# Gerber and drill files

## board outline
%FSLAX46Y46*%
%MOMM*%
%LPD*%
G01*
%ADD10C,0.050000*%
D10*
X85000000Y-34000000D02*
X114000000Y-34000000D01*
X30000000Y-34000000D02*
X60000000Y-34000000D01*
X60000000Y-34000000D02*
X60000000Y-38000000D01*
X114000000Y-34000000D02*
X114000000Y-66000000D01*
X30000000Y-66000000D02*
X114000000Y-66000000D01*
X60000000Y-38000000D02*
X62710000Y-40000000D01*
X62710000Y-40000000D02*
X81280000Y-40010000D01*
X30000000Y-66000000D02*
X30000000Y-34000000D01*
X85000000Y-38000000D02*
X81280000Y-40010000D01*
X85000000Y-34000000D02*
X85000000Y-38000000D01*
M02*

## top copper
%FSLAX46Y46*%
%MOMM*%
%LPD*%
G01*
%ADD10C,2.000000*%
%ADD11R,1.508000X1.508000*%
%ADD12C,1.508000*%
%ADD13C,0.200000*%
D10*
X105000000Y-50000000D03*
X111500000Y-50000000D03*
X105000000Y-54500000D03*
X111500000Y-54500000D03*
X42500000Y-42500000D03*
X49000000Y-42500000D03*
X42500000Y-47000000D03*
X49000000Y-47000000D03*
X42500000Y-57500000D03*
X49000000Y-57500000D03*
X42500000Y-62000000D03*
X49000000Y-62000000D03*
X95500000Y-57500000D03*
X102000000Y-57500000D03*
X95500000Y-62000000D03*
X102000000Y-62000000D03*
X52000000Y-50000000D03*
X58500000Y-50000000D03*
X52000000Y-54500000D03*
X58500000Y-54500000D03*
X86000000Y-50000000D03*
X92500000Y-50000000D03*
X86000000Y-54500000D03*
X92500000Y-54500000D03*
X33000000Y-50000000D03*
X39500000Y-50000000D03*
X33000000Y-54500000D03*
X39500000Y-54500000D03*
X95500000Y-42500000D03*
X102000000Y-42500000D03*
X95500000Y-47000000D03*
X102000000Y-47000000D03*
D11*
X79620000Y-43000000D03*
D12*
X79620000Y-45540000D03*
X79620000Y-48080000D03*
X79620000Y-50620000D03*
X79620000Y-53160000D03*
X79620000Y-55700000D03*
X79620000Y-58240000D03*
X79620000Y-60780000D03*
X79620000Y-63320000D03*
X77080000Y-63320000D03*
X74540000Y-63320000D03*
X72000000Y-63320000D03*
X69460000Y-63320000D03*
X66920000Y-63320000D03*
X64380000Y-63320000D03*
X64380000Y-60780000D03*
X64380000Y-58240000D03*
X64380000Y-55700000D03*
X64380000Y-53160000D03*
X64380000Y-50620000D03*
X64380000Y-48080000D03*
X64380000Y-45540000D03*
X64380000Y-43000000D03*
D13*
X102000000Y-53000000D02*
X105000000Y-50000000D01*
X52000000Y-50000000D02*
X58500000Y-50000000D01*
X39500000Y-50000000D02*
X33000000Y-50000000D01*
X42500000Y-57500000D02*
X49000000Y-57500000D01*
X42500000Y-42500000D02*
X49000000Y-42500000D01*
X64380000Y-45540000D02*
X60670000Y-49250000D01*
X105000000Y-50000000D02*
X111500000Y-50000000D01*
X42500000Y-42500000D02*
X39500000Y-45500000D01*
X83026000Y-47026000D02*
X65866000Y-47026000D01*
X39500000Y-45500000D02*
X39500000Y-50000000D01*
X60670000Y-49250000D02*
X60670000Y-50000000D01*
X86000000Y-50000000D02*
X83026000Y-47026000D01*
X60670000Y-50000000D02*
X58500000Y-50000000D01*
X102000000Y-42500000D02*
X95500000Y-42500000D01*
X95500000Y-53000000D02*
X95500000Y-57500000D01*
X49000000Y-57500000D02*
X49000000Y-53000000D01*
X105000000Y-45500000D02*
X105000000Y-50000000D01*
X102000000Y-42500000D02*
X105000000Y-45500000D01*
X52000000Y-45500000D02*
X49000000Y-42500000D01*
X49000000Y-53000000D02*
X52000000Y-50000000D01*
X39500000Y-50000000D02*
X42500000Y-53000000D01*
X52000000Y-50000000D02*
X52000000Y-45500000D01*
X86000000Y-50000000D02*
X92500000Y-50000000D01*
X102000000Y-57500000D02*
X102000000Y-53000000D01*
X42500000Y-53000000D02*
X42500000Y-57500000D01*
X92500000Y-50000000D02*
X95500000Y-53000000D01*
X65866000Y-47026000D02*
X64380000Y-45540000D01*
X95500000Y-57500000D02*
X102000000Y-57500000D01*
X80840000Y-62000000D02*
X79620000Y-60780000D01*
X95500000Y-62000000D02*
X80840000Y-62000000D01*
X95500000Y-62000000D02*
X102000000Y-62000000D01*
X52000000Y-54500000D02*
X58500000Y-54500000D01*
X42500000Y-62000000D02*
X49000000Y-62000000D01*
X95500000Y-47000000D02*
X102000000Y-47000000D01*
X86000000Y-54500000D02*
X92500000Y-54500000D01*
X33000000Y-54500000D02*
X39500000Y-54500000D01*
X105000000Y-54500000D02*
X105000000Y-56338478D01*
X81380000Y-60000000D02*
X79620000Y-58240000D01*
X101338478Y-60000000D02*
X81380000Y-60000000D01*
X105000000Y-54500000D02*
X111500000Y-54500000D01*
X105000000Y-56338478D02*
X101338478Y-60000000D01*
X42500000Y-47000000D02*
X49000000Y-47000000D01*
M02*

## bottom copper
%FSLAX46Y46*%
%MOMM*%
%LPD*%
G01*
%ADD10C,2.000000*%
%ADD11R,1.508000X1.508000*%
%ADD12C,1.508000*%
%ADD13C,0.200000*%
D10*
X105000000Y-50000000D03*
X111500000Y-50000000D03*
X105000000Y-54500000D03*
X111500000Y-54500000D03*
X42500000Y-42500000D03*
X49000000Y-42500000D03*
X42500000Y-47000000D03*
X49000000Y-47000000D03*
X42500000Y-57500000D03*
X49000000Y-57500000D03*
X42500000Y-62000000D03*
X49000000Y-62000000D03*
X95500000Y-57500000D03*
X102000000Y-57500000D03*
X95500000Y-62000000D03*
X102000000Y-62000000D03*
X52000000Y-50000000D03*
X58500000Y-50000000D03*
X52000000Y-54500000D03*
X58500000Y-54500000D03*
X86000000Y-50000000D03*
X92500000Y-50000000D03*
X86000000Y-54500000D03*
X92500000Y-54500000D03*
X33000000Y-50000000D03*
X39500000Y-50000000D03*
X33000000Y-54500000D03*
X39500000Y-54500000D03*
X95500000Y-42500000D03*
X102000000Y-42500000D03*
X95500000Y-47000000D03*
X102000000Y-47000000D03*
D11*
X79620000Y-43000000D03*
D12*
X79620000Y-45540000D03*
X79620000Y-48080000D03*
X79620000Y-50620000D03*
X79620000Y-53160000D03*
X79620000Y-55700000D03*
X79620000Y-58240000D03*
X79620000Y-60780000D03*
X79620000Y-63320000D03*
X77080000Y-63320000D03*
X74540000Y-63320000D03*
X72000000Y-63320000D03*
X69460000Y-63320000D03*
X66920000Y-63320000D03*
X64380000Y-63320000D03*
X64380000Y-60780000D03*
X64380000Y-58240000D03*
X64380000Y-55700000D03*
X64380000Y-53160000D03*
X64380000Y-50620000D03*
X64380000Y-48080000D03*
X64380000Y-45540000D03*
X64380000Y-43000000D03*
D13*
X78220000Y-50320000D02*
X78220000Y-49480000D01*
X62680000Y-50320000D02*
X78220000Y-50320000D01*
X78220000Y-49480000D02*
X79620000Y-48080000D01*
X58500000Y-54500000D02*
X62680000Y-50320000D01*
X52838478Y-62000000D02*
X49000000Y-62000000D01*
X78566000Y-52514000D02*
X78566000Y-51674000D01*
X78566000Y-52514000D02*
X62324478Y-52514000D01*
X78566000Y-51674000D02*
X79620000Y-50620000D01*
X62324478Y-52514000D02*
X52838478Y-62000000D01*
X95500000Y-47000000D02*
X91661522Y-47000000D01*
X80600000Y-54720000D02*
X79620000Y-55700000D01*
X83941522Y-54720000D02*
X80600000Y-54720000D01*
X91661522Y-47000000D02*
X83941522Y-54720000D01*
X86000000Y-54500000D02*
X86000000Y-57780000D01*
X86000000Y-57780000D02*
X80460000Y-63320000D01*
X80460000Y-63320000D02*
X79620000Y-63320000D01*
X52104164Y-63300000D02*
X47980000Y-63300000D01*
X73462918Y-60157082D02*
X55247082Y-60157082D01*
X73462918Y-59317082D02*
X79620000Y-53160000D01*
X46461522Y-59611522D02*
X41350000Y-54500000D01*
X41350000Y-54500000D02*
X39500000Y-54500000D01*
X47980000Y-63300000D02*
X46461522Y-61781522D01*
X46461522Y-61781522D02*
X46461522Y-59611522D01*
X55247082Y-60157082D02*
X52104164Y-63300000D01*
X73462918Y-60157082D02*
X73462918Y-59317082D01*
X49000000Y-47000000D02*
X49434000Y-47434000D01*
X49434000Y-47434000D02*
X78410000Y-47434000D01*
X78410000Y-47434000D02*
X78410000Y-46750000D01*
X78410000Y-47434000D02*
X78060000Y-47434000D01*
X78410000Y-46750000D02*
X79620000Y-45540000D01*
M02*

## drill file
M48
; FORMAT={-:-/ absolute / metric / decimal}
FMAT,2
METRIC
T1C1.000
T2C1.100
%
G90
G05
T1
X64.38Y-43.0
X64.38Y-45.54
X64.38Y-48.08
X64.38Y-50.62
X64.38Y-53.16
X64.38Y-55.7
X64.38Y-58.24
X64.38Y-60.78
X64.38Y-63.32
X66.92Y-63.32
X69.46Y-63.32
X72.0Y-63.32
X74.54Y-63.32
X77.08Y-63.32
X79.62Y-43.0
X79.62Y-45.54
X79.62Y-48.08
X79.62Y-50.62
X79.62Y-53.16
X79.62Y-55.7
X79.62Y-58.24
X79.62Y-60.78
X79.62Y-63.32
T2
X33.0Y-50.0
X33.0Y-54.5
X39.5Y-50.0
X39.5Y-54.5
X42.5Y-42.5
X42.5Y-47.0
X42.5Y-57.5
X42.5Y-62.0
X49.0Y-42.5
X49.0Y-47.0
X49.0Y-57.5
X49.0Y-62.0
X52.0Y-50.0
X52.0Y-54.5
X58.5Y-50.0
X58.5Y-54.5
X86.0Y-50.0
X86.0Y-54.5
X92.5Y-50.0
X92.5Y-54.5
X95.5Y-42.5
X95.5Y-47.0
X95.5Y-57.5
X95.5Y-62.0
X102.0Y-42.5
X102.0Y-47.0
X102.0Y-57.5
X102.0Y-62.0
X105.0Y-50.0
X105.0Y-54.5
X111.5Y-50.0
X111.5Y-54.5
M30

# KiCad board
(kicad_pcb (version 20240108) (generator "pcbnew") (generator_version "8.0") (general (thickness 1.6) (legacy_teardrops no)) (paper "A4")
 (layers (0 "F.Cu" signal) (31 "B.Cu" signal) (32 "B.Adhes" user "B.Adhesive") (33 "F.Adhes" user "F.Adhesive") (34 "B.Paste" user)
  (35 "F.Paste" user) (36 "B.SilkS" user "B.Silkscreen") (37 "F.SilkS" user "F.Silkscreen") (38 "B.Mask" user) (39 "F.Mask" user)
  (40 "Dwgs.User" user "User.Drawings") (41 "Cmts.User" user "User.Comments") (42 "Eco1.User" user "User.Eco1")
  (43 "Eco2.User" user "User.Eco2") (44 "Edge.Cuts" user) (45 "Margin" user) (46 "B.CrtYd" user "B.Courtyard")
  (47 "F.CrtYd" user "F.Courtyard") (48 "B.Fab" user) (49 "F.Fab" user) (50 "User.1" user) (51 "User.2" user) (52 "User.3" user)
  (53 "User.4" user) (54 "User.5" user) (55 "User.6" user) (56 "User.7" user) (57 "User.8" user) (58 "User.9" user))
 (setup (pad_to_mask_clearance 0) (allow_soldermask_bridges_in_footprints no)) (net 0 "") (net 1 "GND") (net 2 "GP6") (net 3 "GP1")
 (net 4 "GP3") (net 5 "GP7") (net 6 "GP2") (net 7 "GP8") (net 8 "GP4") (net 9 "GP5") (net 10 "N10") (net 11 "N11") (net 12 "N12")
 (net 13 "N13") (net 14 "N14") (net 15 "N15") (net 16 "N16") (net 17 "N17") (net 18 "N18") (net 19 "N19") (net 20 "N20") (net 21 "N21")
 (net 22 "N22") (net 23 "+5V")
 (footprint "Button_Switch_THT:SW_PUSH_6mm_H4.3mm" (layer "F.Cu") (at 105 50)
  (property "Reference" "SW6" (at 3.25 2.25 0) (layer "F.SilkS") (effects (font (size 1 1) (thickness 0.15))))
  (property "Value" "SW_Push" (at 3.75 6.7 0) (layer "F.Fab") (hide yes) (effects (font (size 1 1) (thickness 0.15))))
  (pad "1" thru_hole circle (at 0 0 90) (size 2 2) (drill 1.1) (layers "*.Cu" "*.Mask") (remove_unused_layers no) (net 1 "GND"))
  (pad "1" thru_hole circle (at 6.5 0 90) (size 2 2) (drill 1.1) (layers "*.Cu" "*.Mask") (remove_unused_layers no) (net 1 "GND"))
  (pad "2" thru_hole circle (at 0 4.5 90) (size 2 2) (drill 1.1) (layers "*.Cu" "*.Mask") (remove_unused_layers no) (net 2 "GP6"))
  (pad "2" thru_hole circle (at 6.5 4.5 90) (size 2 2) (drill 1.1) (layers "*.Cu" "*.Mask") (remove_unused_layers no) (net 2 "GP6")))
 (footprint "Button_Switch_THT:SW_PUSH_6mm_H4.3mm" (layer "F.Cu") (at 42.5 42.5)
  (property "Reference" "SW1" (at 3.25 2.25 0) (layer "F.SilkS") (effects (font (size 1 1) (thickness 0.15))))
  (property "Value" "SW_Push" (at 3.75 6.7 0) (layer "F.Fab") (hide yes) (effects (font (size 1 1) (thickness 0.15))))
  (pad "1" thru_hole circle (at 0 0 90) (size 2 2) (drill 1.1) (layers "*.Cu" "*.Mask") (remove_unused_layers no) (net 1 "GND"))
  (pad "1" thru_hole circle (at 6.5 0 90) (size 2 2) (drill 1.1) (layers "*.Cu" "*.Mask") (remove_unused_layers no) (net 1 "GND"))
  (pad "2" thru_hole circle (at 0 4.5 90) (size 2 2) (drill 1.1) (layers "*.Cu" "*.Mask") (remove_unused_layers no) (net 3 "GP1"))
  (pad "2" thru_hole circle (at 6.5 4.5 90) (size 2 2) (drill 1.1) (layers "*.Cu" "*.Mask") (remove_unused_layers no) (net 3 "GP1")))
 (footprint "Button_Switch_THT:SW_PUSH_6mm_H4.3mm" (layer "F.Cu") (at 42.5 57.5)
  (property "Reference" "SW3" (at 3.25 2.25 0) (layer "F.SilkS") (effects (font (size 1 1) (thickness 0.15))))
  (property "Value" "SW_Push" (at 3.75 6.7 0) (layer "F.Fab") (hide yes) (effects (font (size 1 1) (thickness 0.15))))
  (pad "1" thru_hole circle (at 0 0 90) (size 2 2) (drill 1.1) (layers "*.Cu" "*.Mask") (remove_unused_layers no) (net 1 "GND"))
  (pad "1" thru_hole circle (at 6.5 0 90) (size 2 2) (drill 1.1) (layers "*.Cu" "*.Mask") (remove_unused_layers no) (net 1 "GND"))
  (pad "2" thru_hole circle (at 0 4.5 90) (size 2 2) (drill 1.1) (layers "*.Cu" "*.Mask") (remove_unused_layers no) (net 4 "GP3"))
  (pad "2" thru_hole circle (at 6.5 4.5 90) (size 2 2) (drill 1.1) (layers "*.Cu" "*.Mask") (remove_unused_layers no) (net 4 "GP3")))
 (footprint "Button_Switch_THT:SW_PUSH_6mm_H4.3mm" (layer "F.Cu") (at 95.5 57.5)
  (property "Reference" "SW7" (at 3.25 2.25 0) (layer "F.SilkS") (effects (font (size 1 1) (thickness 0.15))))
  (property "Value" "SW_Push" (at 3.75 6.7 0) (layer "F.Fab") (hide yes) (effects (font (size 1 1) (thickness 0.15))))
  (pad "1" thru_hole circle (at 0 0 90) (size 2 2) (drill 1.1) (layers "*.Cu" "*.Mask") (remove_unused_layers no) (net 1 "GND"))
  (pad "1" thru_hole circle (at 6.5 0 90) (size 2 2) (drill 1.1) (layers "*.Cu" "*.Mask") (remove_unused_layers no) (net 1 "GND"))
  (pad "2" thru_hole circle (at 0 4.5 90) (size 2 2) (drill 1.1) (layers "*.Cu" "*.Mask") (remove_unused_layers no) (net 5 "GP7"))
  (pad "2" thru_hole circle (at 6.5 4.5 90) (size 2 2) (drill 1.1) (layers "*.Cu" "*.Mask") (remove_unused_layers no) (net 5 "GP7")))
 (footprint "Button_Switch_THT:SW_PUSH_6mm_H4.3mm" (layer "F.Cu") (at 52 50)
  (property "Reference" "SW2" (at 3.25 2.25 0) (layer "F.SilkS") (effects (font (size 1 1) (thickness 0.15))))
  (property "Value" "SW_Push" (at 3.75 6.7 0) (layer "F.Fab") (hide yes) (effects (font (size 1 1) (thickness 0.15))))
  (pad "1" thru_hole circle (at 0 0 90) (size 2 2) (drill 1.1) (layers "*.Cu" "*.Mask") (remove_unused_layers no) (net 1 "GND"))
  (pad "1" thru_hole circle (at 6.5 0 90) (size 2 2) (drill 1.1) (layers "*.Cu" "*.Mask") (remove_unused_layers no) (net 1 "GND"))
  (pad "2" thru_hole circle (at 0 4.5 90) (size 2 2) (drill 1.1) (layers "*.Cu" "*.Mask") (remove_unused_layers no) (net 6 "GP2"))
  (pad "2" thru_hole circle (at 6.5 4.5 90) (size 2 2) (drill 1.1) (layers "*.Cu" "*.Mask") (remove_unused_layers no) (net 6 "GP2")))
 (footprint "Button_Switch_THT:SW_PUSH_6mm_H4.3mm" (layer "F.Cu") (at 86 50)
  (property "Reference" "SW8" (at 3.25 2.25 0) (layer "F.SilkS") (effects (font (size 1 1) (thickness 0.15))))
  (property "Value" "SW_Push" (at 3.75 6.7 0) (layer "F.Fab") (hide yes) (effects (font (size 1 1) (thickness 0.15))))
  (pad "1" thru_hole circle (at 0 0 90) (size 2 2) (drill 1.1) (layers "*.Cu" "*.Mask") (remove_unused_layers no) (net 1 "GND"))
  (pad "1" thru_hole circle (at 6.5 0 90) (size 2 2) (drill 1.1) (layers "*.Cu" "*.Mask") (remove_unused_layers no) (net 1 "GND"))
  (pad "2" thru_hole circle (at 0 4.5 90) (size 2 2) (drill 1.1) (layers "*.Cu" "*.Mask") (remove_unused_layers no) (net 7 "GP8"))
  (pad "2" thru_hole circle (at 6.5 4.5 90) (size 2 2) (drill 1.1) (layers "*.Cu" "*.Mask") (remove_unused_layers no) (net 7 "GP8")))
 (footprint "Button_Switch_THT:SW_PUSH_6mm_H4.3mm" (layer "F.Cu") (at 33 50)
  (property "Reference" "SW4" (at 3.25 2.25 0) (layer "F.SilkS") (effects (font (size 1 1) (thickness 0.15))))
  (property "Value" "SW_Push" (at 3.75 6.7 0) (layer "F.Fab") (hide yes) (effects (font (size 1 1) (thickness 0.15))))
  (pad "1" thru_hole circle (at 0 0 90) (size 2 2) (drill 1.1) (layers "*.Cu" "*.Mask") (remove_unused_layers no) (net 1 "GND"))
  (pad "1" thru_hole circle (at 6.5 0 90) (size 2 2) (drill 1.1) (layers "*.Cu" "*.Mask") (remove_unused_layers no) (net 1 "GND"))
  (pad "2" thru_hole circle (at 0 4.5 90) (size 2 2) (drill 1.1) (layers "*.Cu" "*.Mask") (remove_unused_layers no) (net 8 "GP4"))
  (pad "2" thru_hole circle (at 6.5 4.5 90) (size 2 2) (drill 1.1) (layers "*.Cu" "*.Mask") (remove_unused_layers no) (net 8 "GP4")))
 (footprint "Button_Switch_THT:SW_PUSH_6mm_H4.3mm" (layer "F.Cu") (at 95.5 42.5)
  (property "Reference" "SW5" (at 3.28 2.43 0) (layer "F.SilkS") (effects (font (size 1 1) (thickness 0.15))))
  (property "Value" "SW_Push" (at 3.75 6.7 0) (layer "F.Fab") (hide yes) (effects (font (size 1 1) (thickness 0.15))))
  (pad "1" thru_hole circle (at 0 0 90) (size 2 2) (drill 1.1) (layers "*.Cu" "*.Mask") (remove_unused_layers no) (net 1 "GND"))
  (pad "1" thru_hole circle (at 6.5 0 90) (size 2 2) (drill 1.1) (layers "*.Cu" "*.Mask") (remove_unused_layers no) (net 1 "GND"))
  (pad "2" thru_hole circle (at 0 4.5 90) (size 2 2) (drill 1.1) (layers "*.Cu" "*.Mask") (remove_unused_layers no) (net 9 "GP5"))
  (pad "2" thru_hole circle (at 6.5 4.5 90) (size 2 2) (drill 1.1) (layers "*.Cu" "*.Mask") (remove_unused_layers no) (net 9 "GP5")))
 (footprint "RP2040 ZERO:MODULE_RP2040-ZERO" (layer "F.Cu") (at 72 53.16)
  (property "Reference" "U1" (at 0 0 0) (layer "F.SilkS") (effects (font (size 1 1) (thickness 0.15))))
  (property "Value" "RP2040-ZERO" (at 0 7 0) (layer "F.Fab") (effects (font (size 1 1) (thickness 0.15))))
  (pad "1" thru_hole rect (at 7.62 -10.16) (size 1.508 1.508) (drill 1) (layers "*.Cu" "*.Mask") (remove_unused_layers no) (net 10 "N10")
   (solder_mask_margin 0.102))
  (pad "2" thru_hole circle (at 7.62 -7.62) (size 1.508 1.508) (drill 1) (layers "*.Cu" "*.Mask") (remove_unused_layers no) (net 3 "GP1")
   (solder_mask_margin 0.102))
  (pad "3" thru_hole circle (at 7.62 -5.08) (size 1.508 1.508) (drill 1) (layers "*.Cu" "*.Mask") (remove_unused_layers no) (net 6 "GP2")
   (solder_mask_margin 0.102))
  (pad "4" thru_hole circle (at 7.62 -2.54) (size 1.508 1.508) (drill 1) (layers "*.Cu" "*.Mask") (remove_unused_layers no) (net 4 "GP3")
   (solder_mask_margin 0.102))
  (pad "5" thru_hole circle (at 7.62 0) (size 1.508 1.508) (drill 1) (layers "*.Cu" "*.Mask") (remove_unused_layers no) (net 8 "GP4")
   (solder_mask_margin 0.102))
  (pad "6" thru_hole circle (at 7.62 2.54) (size 1.508 1.508) (drill 1) (layers "*.Cu" "*.Mask") (remove_unused_layers no) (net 9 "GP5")
   (solder_mask_margin 0.102))
  (pad "7" thru_hole circle (at 7.62 5.08) (size 1.508 1.508) (drill 1) (layers "*.Cu" "*.Mask") (remove_unused_layers no) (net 2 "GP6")
   (solder_mask_margin 0.102))
  (pad "8" thru_hole circle (at 7.62 7.62) (size 1.508 1.508) (drill 1) (layers "*.Cu" "*.Mask") (remove_unused_layers no) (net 5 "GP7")
   (solder_mask_margin 0.102))
  (pad "9" thru_hole circle (at 7.62 10.16) (size 1.508 1.508) (drill 1) (layers "*.Cu" "*.Mask") (remove_unused_layers no) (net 7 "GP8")
   (solder_mask_margin 0.102))
  (pad "10" thru_hole circle (at 5.08 10.16) (size 1.508 1.508) (drill 1) (layers "*.Cu" "*.Mask") (remove_unused_layers no) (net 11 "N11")
   (solder_mask_margin 0.102))
  (pad "11" thru_hole circle (at 2.54 10.16) (size 1.508 1.508) (drill 1) (layers "*.Cu" "*.Mask") (remove_unused_layers no) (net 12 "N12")
   (solder_mask_margin 0.102))
  (pad "12" thru_hole circle (at 0 10.16) (size 1.508 1.508) (drill 1) (layers "*.Cu" "*.Mask") (remove_unused_layers no) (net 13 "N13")
   (solder_mask_margin 0.102))
  (pad "13" thru_hole circle (at -2.54 10.16) (size 1.508 1.508) (drill 1) (layers "*.Cu" "*.Mask") (remove_unused_layers no) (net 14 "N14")
   (solder_mask_margin 0.102))
  (pad "14" thru_hole circle (at -5.08 10.16) (size 1.508 1.508) (drill 1) (layers "*.Cu" "*.Mask") (remove_unused_layers no) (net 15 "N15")
   (solder_mask_margin 0.102))
  (pad "15" thru_hole circle (at -7.62 10.16) (size 1.508 1.508) (drill 1) (layers "*.Cu" "*.Mask") (remove_unused_layers no) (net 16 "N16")
   (solder_mask_margin 0.102))
  (pad "16" thru_hole circle (at -7.62 7.62) (size 1.508 1.508) (drill 1) (layers "*.Cu" "*.Mask") (remove_unused_layers no) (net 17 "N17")
   (solder_mask_margin 0.102))
  (pad "17" thru_hole circle (at -7.62 5.08) (size 1.508 1.508) (drill 1) (layers "*.Cu" "*.Mask") (remove_unused_layers no) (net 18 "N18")
   (solder_mask_margin 0.102))
  (pad "18" thru_hole circle (at -7.62 2.54) (size 1.508 1.508) (drill 1) (layers "*.Cu" "*.Mask") (remove_unused_layers no) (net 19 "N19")
   (solder_mask_margin 0.102))
  (pad "19" thru_hole circle (at -7.62 0) (size 1.508 1.508) (drill 1) (layers "*.Cu" "*.Mask") (remove_unused_layers no) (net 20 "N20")
   (solder_mask_margin 0.102))
  (pad "20" thru_hole circle (at -7.62 -2.54) (size 1.508 1.508) (drill 1) (layers "*.Cu" "*.Mask") (remove_unused_layers no) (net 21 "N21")
   (solder_mask_margin 0.102))
  (pad "21" thru_hole circle (at -7.62 -5.08) (size 1.508 1.508) (drill 1) (layers "*.Cu" "*.Mask") (remove_unused_layers no) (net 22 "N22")
   (solder_mask_margin 0.102))
  (pad "22" thru_hole circle (at -7.62 -7.62) (size 1.508 1.508) (drill 1) (layers "*.Cu" "*.Mask") (remove_unused_layers no) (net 1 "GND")
   (solder_mask_margin 0.102))
  (pad "23" thru_hole circle (at -7.62 -10.16) (size 1.508 1.508) (drill 1) (layers "*.Cu" "*.Mask") (remove_unused_layers no)
   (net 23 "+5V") (solder_mask_margin 0.102)))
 (gr_line (start 85 34) (end 114 34) (stroke (width 0.05) (type default)) (layer "Edge.Cuts"))
 (gr_line (start 30 34) (end 60 34) (stroke (width 0.05) (type default)) (layer "Edge.Cuts"))
 (gr_line (start 60 34) (end 60 38) (stroke (width 0.05) (type default)) (layer "Edge.Cuts"))
 (gr_line (start 114 34) (end 114 66) (stroke (width 0.05) (type default)) (layer "Edge.Cuts"))
 (gr_line (start 30 66) (end 114 66) (stroke (width 0.05) (type default)) (layer "Edge.Cuts"))
 (gr_line (start 60 38) (end 62.71 40) (stroke (width 0.05) (type default)) (layer "Edge.Cuts"))
 (gr_line (start 62.71 40) (end 81.28 40.01) (stroke (width 0.05) (type default)) (layer "Edge.Cuts"))
 (gr_line (start 30 66) (end 30 34) (stroke (width 0.05) (type default)) (layer "Edge.Cuts"))
 (gr_line (start 85 38) (end 81.28 40.01) (stroke (width 0.05) (type default)) (layer "Edge.Cuts"))
 (gr_line (start 85 34) (end 85 38) (stroke (width 0.05) (type default)) (layer "Edge.Cuts"))
 (segment (start 102 53) (end 105 50) (width 0.2) (layer "F.Cu") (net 1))
 (segment (start 52 50) (end 58.5 50) (width 0.2) (layer "F.Cu") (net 1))
 (segment (start 39.5 50) (end 33 50) (width 0.2) (layer "F.Cu") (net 1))
 (segment (start 42.5 57.5) (end 49 57.5) (width 0.2) (layer "F.Cu") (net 1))
 (segment (start 42.5 42.5) (end 49 42.5) (width 0.2) (layer "F.Cu") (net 1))
 (segment (start 64.38 45.54) (end 60.67 49.25) (width 0.2) (layer "F.Cu") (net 1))
 (segment (start 105 50) (end 111.5 50) (width 0.2) (layer "F.Cu") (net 1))
 (segment (start 42.5 42.5) (end 39.5 45.5) (width 0.2) (layer "F.Cu") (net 1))
 (segment (start 83.026 47.026) (end 65.866 47.026) (width 0.2) (layer "F.Cu") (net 1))
 (segment (start 39.5 45.5) (end 39.5 50) (width 0.2) (layer "F.Cu") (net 1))
 (segment (start 60.67 49.25) (end 60.67 50) (width 0.2) (layer "F.Cu") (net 1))
 (segment (start 86 50) (end 83.026 47.026) (width 0.2) (layer "F.Cu") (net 1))
 (segment (start 60.67 50) (end 58.5 50) (width 0.2) (layer "F.Cu") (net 1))
 (segment (start 102 42.5) (end 95.5 42.5) (width 0.2) (layer "F.Cu") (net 1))
 (segment (start 95.5 53) (end 95.5 57.5) (width 0.2) (layer "F.Cu") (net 1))
 (segment (start 49 57.5) (end 49 53) (width 0.2) (layer "F.Cu") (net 1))
 (segment (start 105 45.5) (end 105 50) (width 0.2) (layer "F.Cu") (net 1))
 (segment (start 102 42.5) (end 105 45.5) (width 0.2) (layer "F.Cu") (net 1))
 (segment (start 52 45.5) (end 49 42.5) (width 0.2) (layer "F.Cu") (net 1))
 (segment (start 49 53) (end 52 50) (width 0.2) (layer "F.Cu") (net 1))
 (segment (start 39.5 50) (end 42.5 53) (width 0.2) (layer "F.Cu") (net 1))
 (segment (start 52 50) (end 52 45.5) (width 0.2) (layer "F.Cu") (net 1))
 (segment (start 86 50) (end 92.5 50) (width 0.2) (layer "F.Cu") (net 1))
 (segment (start 102 57.5) (end 102 53) (width 0.2) (layer "F.Cu") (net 1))
 (segment (start 42.5 53) (end 42.5 57.5) (width 0.2) (layer "F.Cu") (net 1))
 (segment (start 92.5 50) (end 95.5 53) (width 0.2) (layer "F.Cu") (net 1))
 (segment (start 65.866 47.026) (end 64.38 45.54) (width 0.2) (layer "F.Cu") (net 1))
 (segment (start 95.5 57.5) (end 102 57.5) (width 0.2) (layer "F.Cu") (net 1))
 (segment (start 80.84 62) (end 79.62 60.78) (width 0.2) (layer "F.Cu") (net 5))
 (segment (start 95.5 62) (end 80.84 62) (width 0.2) (layer "F.Cu") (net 5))
 (segment (start 95.5 62) (end 102 62) (width 0.2) (layer "F.Cu") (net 5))
 (segment (start 52 54.5) (end 58.5 54.5) (width 0.2) (layer "F.Cu") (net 6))
 (segment (start 78.22 50.32) (end 78.22 49.48) (width 0.2) (layer "B.Cu") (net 6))
 (segment (start 62.68 50.32) (end 78.22 50.32) (width 0.2) (layer "B.Cu") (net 6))
 (segment (start 78.22 49.48) (end 79.62 48.08) (width 0.2) (layer "B.Cu") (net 6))
 (segment (start 58.5 54.5) (end 62.68 50.32) (width 0.2) (layer "B.Cu") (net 6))
 (segment (start 42.5 62) (end 49 62) (width 0.2) (layer "F.Cu") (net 4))
 (segment (start 52.838478 62) (end 49 62) (width 0.2) (layer "B.Cu") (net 4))
 (segment (start 78.566 52.514) (end 78.566 51.674) (width 0.2) (layer "B.Cu") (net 4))
 (segment (start 78.566 52.514) (end 62.324478 52.514) (width 0.2) (layer "B.Cu") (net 4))
 (segment (start 78.566 51.674) (end 79.62 50.62) (width 0.2) (layer "B.Cu") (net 4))
 (segment (start 62.324478 52.514) (end 52.838478 62) (width 0.2) (layer "B.Cu") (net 4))
 (segment (start 95.5 47) (end 102 47) (width 0.2) (layer "F.Cu") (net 9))
 (segment (start 95.5 47) (end 91.661522 47) (width 0.2) (layer "B.Cu") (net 9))
 (segment (start 80.6 54.72) (end 79.62 55.7) (width 0.2) (layer "B.Cu") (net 9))
 (segment (start 83.941522 54.72) (end 80.6 54.72) (width 0.2) (layer "B.Cu") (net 9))
 (segment (start 91.661522 47) (end 83.941522 54.72) (width 0.2) (layer "B.Cu") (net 9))
 (segment (start 86 54.5) (end 92.5 54.5) (width 0.2) (layer "F.Cu") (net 7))
 (segment (start 86 54.5) (end 86 57.78) (width 0.2) (layer "B.Cu") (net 7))
 (segment (start 86 57.78) (end 80.46 63.32) (width 0.2) (layer "B.Cu") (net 7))
 (segment (start 80.46 63.32) (end 79.62 63.32) (width 0.2) (layer "B.Cu") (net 7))
 (segment (start 33 54.5) (end 39.5 54.5) (width 0.2) (layer "F.Cu") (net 8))
 (segment (start 52.104164 63.3) (end 47.98 63.3) (width 0.2) (layer "B.Cu") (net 8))
 (segment (start 73.462918 60.157082) (end 55.247082 60.157082) (width 0.2) (layer "B.Cu") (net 8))
 (segment (start 73.462918 59.317082) (end 79.62 53.16) (width 0.2) (layer "B.Cu") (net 8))
 (segment (start 46.461522 59.611522) (end 41.35 54.5) (width 0.2) (layer "B.Cu") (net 8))
 (segment (start 41.35 54.5) (end 39.5 54.5) (width 0.2) (layer "B.Cu") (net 8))
 (segment (start 47.98 63.3) (end 46.461522 61.781522) (width 0.2) (layer "B.Cu") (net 8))
 (segment (start 46.461522 61.781522) (end 46.461522 59.611522) (width 0.2) (layer "B.Cu") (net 8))
 (segment (start 55.247082 60.157082) (end 52.104164 63.3) (width 0.2) (layer "B.Cu") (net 8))
 (segment (start 73.462918 60.157082) (end 73.462918 59.317082) (width 0.2) (layer "B.Cu") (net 8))
 (segment (start 105 54.5) (end 105 56.338478) (width 0.2) (layer "F.Cu") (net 2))
 (segment (start 81.38 60) (end 79.62 58.24) (width 0.2) (layer "F.Cu") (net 2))
 (segment (start 101.338478 60) (end 81.38 60) (width 0.2) (layer "F.Cu") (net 2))
 (segment (start 105 54.5) (end 111.5 54.5) (width 0.2) (layer "F.Cu") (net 2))
 (segment (start 105 56.338478) (end 101.338478 60) (width 0.2) (layer "F.Cu") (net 2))
 (segment (start 42.5 47) (end 49 47) (width 0.2) (layer "F.Cu") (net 3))
 (segment (start 49 47) (end 49.434 47.434) (width 0.2) (layer "B.Cu") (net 3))
 (segment (start 49.434 47.434) (end 78.41 47.434) (width 0.2) (layer "B.Cu") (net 3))
 (segment (start 78.41 47.434) (end 78.41 46.75) (width 0.2) (layer "B.Cu") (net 3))
 (segment (start 78.41 47.434) (end 78.06 47.434) (width 0.2) (layer "B.Cu") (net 3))
 (segment (start 78.41 46.75) (end 79.62 45.54) (width 0.2) (layer "B.Cu") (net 3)))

